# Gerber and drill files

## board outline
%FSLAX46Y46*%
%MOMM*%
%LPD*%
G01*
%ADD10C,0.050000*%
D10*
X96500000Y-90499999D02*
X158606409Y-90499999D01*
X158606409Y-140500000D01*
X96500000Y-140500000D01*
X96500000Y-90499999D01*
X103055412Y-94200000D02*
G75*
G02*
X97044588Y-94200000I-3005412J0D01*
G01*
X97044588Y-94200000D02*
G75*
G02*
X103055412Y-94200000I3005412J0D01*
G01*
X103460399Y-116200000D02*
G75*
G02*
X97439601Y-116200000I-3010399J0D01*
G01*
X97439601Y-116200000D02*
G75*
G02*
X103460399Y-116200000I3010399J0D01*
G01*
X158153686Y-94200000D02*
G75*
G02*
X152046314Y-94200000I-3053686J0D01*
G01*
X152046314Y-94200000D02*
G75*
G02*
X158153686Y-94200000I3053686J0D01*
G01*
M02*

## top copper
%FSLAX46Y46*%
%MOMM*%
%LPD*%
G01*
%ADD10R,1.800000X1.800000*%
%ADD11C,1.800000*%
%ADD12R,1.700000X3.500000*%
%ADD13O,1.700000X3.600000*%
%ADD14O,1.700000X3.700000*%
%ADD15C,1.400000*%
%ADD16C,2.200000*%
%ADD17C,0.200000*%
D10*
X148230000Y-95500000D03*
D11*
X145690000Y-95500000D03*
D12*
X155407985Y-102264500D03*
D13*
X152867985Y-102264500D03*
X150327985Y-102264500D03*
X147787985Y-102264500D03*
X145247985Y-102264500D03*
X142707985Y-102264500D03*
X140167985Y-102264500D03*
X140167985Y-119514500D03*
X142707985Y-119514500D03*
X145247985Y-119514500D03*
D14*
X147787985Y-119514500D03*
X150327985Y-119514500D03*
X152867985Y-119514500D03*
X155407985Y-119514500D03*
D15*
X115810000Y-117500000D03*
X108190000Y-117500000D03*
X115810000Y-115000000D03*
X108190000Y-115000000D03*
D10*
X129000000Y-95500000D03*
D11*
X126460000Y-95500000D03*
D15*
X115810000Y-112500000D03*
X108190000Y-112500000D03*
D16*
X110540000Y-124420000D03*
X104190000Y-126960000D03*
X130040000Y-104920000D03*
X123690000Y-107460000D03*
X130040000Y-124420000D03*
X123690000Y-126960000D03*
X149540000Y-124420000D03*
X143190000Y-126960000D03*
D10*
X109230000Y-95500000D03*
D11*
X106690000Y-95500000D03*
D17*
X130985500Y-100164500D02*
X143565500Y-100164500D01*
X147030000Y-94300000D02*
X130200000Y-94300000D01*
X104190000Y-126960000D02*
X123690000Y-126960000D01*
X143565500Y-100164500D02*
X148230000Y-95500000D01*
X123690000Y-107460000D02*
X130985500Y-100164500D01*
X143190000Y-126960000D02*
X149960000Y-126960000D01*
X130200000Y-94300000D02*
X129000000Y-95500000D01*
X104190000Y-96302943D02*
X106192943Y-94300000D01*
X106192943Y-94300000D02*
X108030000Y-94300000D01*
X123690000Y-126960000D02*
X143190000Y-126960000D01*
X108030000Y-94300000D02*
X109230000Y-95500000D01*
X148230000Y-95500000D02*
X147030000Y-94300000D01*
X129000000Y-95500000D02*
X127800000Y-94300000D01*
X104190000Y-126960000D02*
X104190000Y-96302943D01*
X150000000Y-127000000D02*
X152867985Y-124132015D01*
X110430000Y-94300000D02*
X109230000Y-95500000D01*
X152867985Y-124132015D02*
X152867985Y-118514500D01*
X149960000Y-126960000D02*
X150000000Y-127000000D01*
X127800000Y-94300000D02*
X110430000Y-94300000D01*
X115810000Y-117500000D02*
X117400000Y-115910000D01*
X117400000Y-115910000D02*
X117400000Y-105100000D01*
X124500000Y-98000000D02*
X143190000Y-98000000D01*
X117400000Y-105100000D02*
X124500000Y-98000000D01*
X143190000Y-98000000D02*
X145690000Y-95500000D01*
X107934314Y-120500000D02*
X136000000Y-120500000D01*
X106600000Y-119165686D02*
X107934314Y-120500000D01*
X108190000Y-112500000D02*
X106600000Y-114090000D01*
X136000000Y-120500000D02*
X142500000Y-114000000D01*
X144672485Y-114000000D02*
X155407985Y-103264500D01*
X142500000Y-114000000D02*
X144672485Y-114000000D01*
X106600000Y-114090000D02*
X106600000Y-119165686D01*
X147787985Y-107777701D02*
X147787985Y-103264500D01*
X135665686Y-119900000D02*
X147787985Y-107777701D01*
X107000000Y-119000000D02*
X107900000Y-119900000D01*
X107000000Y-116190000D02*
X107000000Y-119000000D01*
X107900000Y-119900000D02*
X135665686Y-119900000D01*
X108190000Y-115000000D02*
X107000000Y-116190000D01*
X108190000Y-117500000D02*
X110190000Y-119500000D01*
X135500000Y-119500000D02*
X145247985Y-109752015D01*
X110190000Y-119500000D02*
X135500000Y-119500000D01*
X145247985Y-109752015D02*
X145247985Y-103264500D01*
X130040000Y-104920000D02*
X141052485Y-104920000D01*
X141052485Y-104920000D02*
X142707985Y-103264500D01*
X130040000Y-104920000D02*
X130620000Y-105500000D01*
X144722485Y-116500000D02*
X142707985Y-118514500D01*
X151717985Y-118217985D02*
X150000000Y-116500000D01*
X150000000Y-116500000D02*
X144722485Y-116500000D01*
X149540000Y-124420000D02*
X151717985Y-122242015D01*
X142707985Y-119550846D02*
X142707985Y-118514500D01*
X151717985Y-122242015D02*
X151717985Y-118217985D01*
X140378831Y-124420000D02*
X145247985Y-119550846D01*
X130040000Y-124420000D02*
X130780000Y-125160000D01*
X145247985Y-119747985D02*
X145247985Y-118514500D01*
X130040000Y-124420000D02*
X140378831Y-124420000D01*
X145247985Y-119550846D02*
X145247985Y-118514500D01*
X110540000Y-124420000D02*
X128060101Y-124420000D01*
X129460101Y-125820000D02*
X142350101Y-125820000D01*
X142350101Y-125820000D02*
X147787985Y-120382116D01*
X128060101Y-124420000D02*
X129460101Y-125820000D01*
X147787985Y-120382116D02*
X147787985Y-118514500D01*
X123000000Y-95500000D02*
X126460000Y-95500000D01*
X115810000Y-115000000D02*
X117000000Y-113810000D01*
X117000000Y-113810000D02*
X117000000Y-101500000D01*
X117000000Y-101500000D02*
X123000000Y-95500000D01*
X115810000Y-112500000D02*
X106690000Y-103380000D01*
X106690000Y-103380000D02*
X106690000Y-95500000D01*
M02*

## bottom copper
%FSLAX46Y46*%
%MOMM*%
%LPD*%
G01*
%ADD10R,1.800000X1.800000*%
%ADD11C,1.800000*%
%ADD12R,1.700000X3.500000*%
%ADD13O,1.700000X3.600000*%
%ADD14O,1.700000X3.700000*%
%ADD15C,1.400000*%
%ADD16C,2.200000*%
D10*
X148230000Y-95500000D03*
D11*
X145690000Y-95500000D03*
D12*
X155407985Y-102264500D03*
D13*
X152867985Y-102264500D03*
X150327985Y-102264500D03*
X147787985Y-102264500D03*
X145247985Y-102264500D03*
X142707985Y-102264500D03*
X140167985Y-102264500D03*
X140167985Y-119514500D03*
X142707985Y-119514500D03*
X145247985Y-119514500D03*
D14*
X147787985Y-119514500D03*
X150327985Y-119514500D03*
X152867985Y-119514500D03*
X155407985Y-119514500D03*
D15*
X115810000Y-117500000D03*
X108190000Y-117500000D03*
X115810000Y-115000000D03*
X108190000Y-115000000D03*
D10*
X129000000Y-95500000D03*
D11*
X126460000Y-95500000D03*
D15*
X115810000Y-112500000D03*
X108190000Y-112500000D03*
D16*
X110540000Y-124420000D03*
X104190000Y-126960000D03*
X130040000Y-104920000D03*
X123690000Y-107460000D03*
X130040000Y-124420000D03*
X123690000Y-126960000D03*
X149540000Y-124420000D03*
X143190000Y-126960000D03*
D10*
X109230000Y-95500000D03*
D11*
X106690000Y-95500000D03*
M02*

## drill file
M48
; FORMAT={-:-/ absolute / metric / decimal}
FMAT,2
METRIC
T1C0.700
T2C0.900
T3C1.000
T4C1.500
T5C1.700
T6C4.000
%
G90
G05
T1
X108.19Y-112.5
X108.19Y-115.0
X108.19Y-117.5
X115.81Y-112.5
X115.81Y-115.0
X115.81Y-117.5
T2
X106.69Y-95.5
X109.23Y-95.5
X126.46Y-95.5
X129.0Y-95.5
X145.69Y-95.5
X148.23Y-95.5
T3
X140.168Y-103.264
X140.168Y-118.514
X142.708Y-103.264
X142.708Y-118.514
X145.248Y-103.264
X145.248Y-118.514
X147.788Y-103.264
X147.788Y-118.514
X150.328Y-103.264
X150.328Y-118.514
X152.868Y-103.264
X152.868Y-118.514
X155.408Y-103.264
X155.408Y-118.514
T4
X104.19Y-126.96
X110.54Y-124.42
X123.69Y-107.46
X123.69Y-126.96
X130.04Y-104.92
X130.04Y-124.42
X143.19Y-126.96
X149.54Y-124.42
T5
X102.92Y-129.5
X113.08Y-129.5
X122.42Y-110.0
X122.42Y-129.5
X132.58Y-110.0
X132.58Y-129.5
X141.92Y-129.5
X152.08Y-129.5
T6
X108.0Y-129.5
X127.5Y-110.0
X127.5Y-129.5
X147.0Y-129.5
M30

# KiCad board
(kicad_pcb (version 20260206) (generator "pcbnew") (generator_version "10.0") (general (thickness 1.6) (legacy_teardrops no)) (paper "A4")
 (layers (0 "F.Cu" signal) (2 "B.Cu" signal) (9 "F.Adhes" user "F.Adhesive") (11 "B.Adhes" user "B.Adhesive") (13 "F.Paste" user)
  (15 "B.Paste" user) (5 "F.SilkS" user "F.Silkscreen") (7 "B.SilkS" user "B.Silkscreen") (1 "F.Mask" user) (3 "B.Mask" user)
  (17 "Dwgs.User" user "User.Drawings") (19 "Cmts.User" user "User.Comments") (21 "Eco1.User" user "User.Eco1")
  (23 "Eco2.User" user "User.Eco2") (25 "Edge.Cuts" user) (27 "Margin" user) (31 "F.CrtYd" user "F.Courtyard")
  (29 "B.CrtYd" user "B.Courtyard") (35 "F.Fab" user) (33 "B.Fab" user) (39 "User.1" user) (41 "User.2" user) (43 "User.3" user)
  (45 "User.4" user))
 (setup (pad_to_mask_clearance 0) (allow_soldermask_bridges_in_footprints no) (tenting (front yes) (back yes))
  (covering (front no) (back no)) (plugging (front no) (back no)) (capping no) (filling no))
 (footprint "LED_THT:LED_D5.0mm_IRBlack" (layer "F.Cu") (at 148.23 95.5 180)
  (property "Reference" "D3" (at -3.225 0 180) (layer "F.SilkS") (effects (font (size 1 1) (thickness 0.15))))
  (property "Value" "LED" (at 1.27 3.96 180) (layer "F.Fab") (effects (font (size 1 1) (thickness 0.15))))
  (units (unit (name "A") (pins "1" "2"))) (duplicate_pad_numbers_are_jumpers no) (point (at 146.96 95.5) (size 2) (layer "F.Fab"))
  (pad "1" thru_hole rect (at 0 0 180) (size 1.8 1.8) (drill 0.9) (layers "*.Cu" "*.Mask") (remove_unused_layers no) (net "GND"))
  (pad "2" thru_hole circle (at 2.54 0 180) (size 1.8 1.8) (drill 0.9) (layers "*.Cu" "*.Mask") (remove_unused_layers no) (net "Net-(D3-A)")))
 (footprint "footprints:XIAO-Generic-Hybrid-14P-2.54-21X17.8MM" (layer "F.Cu") (at 147.787985 110.8895 -90)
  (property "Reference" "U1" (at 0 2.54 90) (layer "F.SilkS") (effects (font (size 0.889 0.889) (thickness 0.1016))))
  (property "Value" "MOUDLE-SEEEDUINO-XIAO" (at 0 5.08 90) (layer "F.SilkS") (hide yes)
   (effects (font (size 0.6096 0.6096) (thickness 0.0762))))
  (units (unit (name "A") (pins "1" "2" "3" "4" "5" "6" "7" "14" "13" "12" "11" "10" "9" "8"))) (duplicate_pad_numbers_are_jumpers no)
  (pad "1" thru_hole rect (at -7.625 -7.62 270) (size 3.5 1.7) (drill 1 (offset -1 0)) (layers "*.Cu" "*.Mask") (remove_unused_layers no)
   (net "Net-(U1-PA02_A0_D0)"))
  (pad "2" thru_hole oval (at -7.625 -5.08 270) (size 3.6 1.7) (drill 1 (offset -1 0)) (layers "*.Cu" "*.Mask") (remove_unused_layers no)
   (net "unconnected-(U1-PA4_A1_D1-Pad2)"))
  (pad "3" thru_hole oval (at -7.625 -2.54 270) (size 3.6 1.7) (drill 1 (offset -1 0)) (layers "*.Cu" "*.Mask") (remove_unused_layers no)
   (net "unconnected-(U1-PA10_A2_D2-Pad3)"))
  (pad "4" thru_hole oval (at -7.625 0 270) (size 3.6 1.7) (drill 1 (offset -1 0)) (layers "*.Cu" "*.Mask") (remove_unused_layers no)
   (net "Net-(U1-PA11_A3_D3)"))
  (pad "5" thru_hole oval (at -7.625 2.54 270) (size 3.6 1.7) (drill 1 (offset -1 0)) (layers "*.Cu" "*.Mask") (remove_unused_layers no)
   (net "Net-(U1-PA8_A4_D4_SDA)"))
  (pad "6" thru_hole oval (at -7.625 5.08 90) (size 3.6 1.7) (drill 1 (offset 1 0)) (layers "*.Cu" "*.Mask") (remove_unused_layers no)
   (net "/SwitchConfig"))
  (pad "7" thru_hole oval (at -7.625 7.62 270) (size 3.6 1.7) (drill 1 (offset -1 0)) (layers "*.Cu" "*.Mask") (remove_unused_layers no)
   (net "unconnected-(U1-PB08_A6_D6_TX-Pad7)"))
  (pad "8" thru_hole oval (at 7.625 7.62 270) (size 3.6 1.7) (drill 1 (offset 1 0)) (layers "*.Cu" "*.Mask") (remove_unused_layers no)
   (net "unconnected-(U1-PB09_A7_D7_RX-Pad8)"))
  (pad "9" thru_hole oval (at 7.625 5.08 270) (size 3.6 1.7) (drill 1 (offset 1 0)) (layers "*.Cu" "*.Mask") (remove_unused_layers no)
   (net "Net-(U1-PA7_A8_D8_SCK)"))
  (pad "10" thru_hole oval (at 7.625 2.54 270) (size 3.6 1.7) (drill 1 (offset 1 0)) (layers "*.Cu" "*.Mask") (remove_unused_layers no)
   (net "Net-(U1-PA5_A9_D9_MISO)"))
  (pad "11" thru_hole oval (at 7.625 0 270) (size 3.7 1.7) (drill 1 (offset 1 0)) (layers "*.Cu" "*.Mask") (remove_unused_layers no)
   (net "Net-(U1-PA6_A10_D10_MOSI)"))
  (pad "12" thru_hole oval (at 7.625 -2.54 270) (size 3.7 1.7) (drill 1 (offset 1 0)) (layers "*.Cu" "*.Mask") (remove_unused_layers no)
   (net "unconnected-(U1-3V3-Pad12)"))
  (pad "13" thru_hole oval (at 7.625 -5.08 270) (size 3.7 1.7) (drill 1 (offset 1 0)) (layers "*.Cu" "*.Mask") (remove_unused_layers no)
   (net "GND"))
  (pad "14" thru_hole oval (at 7.625 -7.62 270) (size 3.7 1.7) (drill 1 (offset 1 0)) (layers "*.Cu" "*.Mask") (remove_unused_layers no)
   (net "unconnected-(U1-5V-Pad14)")))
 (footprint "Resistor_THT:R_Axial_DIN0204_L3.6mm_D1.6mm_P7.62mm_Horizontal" (layer "F.Cu") (at 115.81 117.5 180)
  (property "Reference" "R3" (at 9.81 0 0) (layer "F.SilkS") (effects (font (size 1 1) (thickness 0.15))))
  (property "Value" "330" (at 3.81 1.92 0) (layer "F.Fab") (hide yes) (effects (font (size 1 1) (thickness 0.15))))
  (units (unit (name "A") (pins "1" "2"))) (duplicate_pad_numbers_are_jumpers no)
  (pad "1" thru_hole circle (at 0 0 180) (size 1.4 1.4) (drill 0.7) (layers "*.Cu" "*.Mask") (remove_unused_layers no) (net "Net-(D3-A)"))
  (pad "2" thru_hole circle (at 7.62 0 180) (size 1.4 1.4) (drill 0.7) (layers "*.Cu" "*.Mask") (remove_unused_layers no)
   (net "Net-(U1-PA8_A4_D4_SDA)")))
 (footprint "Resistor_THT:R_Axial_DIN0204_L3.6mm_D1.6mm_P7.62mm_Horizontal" (layer "F.Cu") (at 115.81 115 180)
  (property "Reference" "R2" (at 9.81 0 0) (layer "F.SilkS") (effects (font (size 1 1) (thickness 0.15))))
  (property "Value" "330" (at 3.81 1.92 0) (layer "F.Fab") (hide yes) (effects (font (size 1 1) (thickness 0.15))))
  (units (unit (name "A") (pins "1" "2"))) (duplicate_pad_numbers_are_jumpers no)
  (pad "1" thru_hole circle (at 0 0 180) (size 1.4 1.4) (drill 0.7) (layers "*.Cu" "*.Mask") (remove_unused_layers no) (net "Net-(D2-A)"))
  (pad "2" thru_hole circle (at 7.62 0 180) (size 1.4 1.4) (drill 0.7) (layers "*.Cu" "*.Mask") (remove_unused_layers no)
   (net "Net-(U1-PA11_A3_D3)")))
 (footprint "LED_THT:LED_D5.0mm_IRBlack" (layer "F.Cu") (at 129 95.5 180)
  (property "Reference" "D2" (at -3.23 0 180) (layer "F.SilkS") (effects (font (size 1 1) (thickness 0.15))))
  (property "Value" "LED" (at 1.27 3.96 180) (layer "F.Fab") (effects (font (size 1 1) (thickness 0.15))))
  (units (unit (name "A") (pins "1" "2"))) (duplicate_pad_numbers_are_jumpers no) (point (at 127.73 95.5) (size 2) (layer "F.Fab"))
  (pad "1" thru_hole rect (at 0 0 180) (size 1.8 1.8) (drill 0.9) (layers "*.Cu" "*.Mask") (remove_unused_layers no) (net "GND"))
  (pad "2" thru_hole circle (at 2.54 0 180) (size 1.8 1.8) (drill 0.9) (layers "*.Cu" "*.Mask") (remove_unused_layers no) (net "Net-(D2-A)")))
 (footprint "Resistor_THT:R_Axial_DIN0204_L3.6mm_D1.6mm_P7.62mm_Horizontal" (layer "F.Cu") (at 115.81 112.5 180)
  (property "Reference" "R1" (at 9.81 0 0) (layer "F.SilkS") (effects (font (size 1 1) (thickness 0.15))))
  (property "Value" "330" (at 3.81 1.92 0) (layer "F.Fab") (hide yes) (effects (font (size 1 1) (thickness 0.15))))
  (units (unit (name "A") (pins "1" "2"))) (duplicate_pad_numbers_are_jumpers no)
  (pad "1" thru_hole circle (at 0 0 180) (size 1.4 1.4) (drill 0.7) (layers "*.Cu" "*.Mask") (remove_unused_layers no) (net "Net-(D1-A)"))
  (pad "2" thru_hole circle (at 7.62 0 180) (size 1.4 1.4) (drill 0.7) (layers "*.Cu" "*.Mask") (remove_unused_layers no)
   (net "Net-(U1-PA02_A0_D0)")))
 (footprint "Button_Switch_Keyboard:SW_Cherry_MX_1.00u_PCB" (layer "F.Cu") (at 110.54 124.42)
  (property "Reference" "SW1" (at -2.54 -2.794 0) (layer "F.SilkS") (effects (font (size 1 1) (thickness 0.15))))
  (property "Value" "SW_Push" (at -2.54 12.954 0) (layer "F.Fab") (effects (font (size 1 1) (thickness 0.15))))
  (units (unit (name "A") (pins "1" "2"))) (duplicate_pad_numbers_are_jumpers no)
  (pad "" np_thru_hole circle (at -7.62 5.08) (size 1.7 1.7) (drill 1.7) (layers "*.Cu" "*.Mask"))
  (pad "" np_thru_hole circle (at -2.54 5.08) (size 4 4) (drill 4) (layers "*.Cu" "*.Mask"))
  (pad "" np_thru_hole circle (at 2.54 5.08) (size 1.7 1.7) (drill 1.7) (layers "*.Cu" "*.Mask"))
  (pad "1" thru_hole circle (at 0 0) (size 2.2 2.2) (drill 1.5) (layers "*.Cu" "*.Mask") (remove_unused_layers no)
   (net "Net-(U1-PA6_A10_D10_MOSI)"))
  (pad "2" thru_hole circle (at -6.35 2.54) (size 2.2 2.2) (drill 1.5) (layers "*.Cu" "*.Mask") (remove_unused_layers no) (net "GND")))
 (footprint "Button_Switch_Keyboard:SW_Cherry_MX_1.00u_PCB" (layer "F.Cu") (at 130.04 104.92)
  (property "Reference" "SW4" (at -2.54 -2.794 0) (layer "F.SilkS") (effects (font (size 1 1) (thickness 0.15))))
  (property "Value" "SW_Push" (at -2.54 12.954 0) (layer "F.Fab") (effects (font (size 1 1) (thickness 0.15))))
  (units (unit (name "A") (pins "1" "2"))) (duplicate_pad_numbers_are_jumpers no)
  (pad "" np_thru_hole circle (at -7.62 5.08) (size 1.7 1.7) (drill 1.7) (layers "*.Cu" "*.Mask"))
  (pad "" np_thru_hole circle (at -2.54 5.08) (size 4 4) (drill 4) (layers "*.Cu" "*.Mask"))
  (pad "" np_thru_hole circle (at 2.54 5.08) (size 1.7 1.7) (drill 1.7) (layers "*.Cu" "*.Mask"))
  (pad "1" thru_hole circle (at 0 0) (size 2.2 2.2) (drill 1.5) (layers "*.Cu" "*.Mask") (remove_unused_layers no) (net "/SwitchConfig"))
  (pad "2" thru_hole circle (at -6.35 2.54) (size 2.2 2.2) (drill 1.5) (layers "*.Cu" "*.Mask") (remove_unused_layers no) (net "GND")))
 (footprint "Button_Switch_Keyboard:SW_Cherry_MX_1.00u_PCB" (layer "F.Cu") (at 130.04 124.42)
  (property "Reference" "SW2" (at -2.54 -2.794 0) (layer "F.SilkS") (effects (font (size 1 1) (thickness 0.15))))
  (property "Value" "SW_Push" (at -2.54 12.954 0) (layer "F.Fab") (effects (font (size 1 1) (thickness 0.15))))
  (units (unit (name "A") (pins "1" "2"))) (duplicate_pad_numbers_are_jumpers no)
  (pad "" np_thru_hole circle (at -7.62 5.08) (size 1.7 1.7) (drill 1.7) (layers "*.Cu" "*.Mask"))
  (pad "" np_thru_hole circle (at -2.54 5.08) (size 4 4) (drill 4) (layers "*.Cu" "*.Mask"))
  (pad "" np_thru_hole circle (at 2.54 5.08) (size 1.7 1.7) (drill 1.7) (layers "*.Cu" "*.Mask"))
  (pad "1" thru_hole circle (at 0 0) (size 2.2 2.2) (drill 1.5) (layers "*.Cu" "*.Mask") (remove_unused_layers no)
   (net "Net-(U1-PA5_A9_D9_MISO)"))
  (pad "2" thru_hole circle (at -6.35 2.54) (size 2.2 2.2) (drill 1.5) (layers "*.Cu" "*.Mask") (remove_unused_layers no) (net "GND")))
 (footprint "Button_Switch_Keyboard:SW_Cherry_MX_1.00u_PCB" (layer "F.Cu") (at 149.54 124.42)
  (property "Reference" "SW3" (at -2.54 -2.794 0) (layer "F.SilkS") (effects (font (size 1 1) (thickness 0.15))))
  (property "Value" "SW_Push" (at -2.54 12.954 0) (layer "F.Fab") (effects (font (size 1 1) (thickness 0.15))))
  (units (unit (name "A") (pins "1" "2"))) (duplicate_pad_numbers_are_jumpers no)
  (pad "" np_thru_hole circle (at -7.62 5.08) (size 1.7 1.7) (drill 1.7) (layers "*.Cu" "*.Mask"))
  (pad "" np_thru_hole circle (at -2.54 5.08) (size 4 4) (drill 4) (layers "*.Cu" "*.Mask"))
  (pad "" np_thru_hole circle (at 2.54 5.08) (size 1.7 1.7) (drill 1.7) (layers "*.Cu" "*.Mask"))
  (pad "1" thru_hole circle (at 0 0) (size 2.2 2.2) (drill 1.5) (layers "*.Cu" "*.Mask") (remove_unused_layers no)
   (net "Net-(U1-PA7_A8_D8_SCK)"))
  (pad "2" thru_hole circle (at -6.35 2.54) (size 2.2 2.2) (drill 1.5) (layers "*.Cu" "*.Mask") (remove_unused_layers no) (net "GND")))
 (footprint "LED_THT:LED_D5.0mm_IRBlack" (layer "F.Cu") (at 109.23 95.5 180)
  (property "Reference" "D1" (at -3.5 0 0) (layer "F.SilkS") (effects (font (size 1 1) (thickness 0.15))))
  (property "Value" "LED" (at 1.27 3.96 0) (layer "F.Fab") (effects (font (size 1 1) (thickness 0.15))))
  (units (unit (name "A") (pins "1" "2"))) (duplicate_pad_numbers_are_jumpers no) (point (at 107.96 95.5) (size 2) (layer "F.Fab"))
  (pad "1" thru_hole rect (at 0 0 180) (size 1.8 1.8) (drill 0.9) (layers "*.Cu" "*.Mask") (remove_unused_layers no) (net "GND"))
  (pad "2" thru_hole circle (at 2.54 0 180) (size 1.8 1.8) (drill 0.9) (layers "*.Cu" "*.Mask") (remove_unused_layers no) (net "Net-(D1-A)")))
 (gr_rect (start 96.5 90.499999) (end 158.606409 140.5) (stroke (width 0.05) (type default)) (fill no) (layer "Edge.Cuts"))
 (gr_circle (center 100.05 94.2) (end 102.15 96.35) (stroke (width 0.05) (type default)) (fill no) (layer "Edge.Cuts"))
 (gr_circle (center 100.45 116.2) (end 102.45 113.95) (stroke (width 0.05) (type default)) (fill no) (layer "Edge.Cuts"))
 (gr_circle (center 155.1 94.2) (end 157.45 92.25) (stroke (width 0.05) (type default)) (fill no) (layer "Edge.Cuts"))
 (segment (start 130.9855 100.1645) (end 143.5655 100.1645) (width 0.2) (layer "F.Cu") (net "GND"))
 (segment (start 147.03 94.3) (end 130.2 94.3) (width 0.2) (layer "F.Cu") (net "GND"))
 (segment (start 104.19 126.96) (end 123.69 126.96) (width 0.2) (layer "F.Cu") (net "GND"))
 (segment (start 143.5655 100.1645) (end 148.23 95.5) (width 0.2) (layer "F.Cu") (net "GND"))
 (segment (start 123.69 107.46) (end 130.9855 100.1645) (width 0.2) (layer "F.Cu") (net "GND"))
 (segment (start 143.19 126.96) (end 149.96 126.96) (width 0.2) (layer "F.Cu") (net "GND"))
 (segment (start 130.2 94.3) (end 129 95.5) (width 0.2) (layer "F.Cu") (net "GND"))
 (segment (start 104.19 96.302943) (end 106.192943 94.3) (width 0.2) (layer "F.Cu") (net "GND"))
 (segment (start 106.192943 94.3) (end 108.03 94.3) (width 0.2) (layer "F.Cu") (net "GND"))
 (segment (start 123.69 126.96) (end 143.19 126.96) (width 0.2) (layer "F.Cu") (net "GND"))
 (segment (start 108.03 94.3) (end 109.23 95.5) (width 0.2) (layer "F.Cu") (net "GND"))
 (segment (start 148.23 95.5) (end 147.03 94.3) (width 0.2) (layer "F.Cu") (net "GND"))
 (segment (start 129 95.5) (end 127.8 94.3) (width 0.2) (layer "F.Cu") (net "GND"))
 (segment (start 104.19 126.96) (end 104.19 96.302943) (width 0.2) (layer "F.Cu") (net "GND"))
 (segment (start 150 127) (end 152.867985 124.132015) (width 0.2) (layer "F.Cu") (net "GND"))
 (segment (start 110.43 94.3) (end 109.23 95.5) (width 0.2) (layer "F.Cu") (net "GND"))
 (segment (start 152.867985 124.132015) (end 152.867985 118.5145) (width 0.2) (layer "F.Cu") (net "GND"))
 (segment (start 149.96 126.96) (end 150 127) (width 0.2) (layer "F.Cu") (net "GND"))
 (segment (start 127.8 94.3) (end 110.43 94.3) (width 0.2) (layer "F.Cu") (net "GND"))
 (segment (start 115.81 117.5) (end 117.4 115.91) (width 0.2) (layer "F.Cu") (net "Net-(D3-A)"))
 (segment (start 117.4 115.91) (end 117.4 105.1) (width 0.2) (layer "F.Cu") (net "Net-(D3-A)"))
 (segment (start 124.5 98) (end 143.19 98) (width 0.2) (layer "F.Cu") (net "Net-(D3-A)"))
 (segment (start 117.4 105.1) (end 124.5 98) (width 0.2) (layer "F.Cu") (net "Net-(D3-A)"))
 (segment (start 143.19 98) (end 145.69 95.5) (width 0.2) (layer "F.Cu") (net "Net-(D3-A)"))
 (segment (start 107.934314 120.5) (end 136 120.5) (width 0.2) (layer "F.Cu") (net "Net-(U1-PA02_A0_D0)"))
 (segment (start 106.6 119.165686) (end 107.934314 120.5) (width 0.2) (layer "F.Cu") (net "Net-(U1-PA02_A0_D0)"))
 (segment (start 108.19 112.5) (end 106.6 114.09) (width 0.2) (layer "F.Cu") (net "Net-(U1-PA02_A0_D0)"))
 (segment (start 136 120.5) (end 142.5 114) (width 0.2) (layer "F.Cu") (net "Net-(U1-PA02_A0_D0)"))
 (segment (start 144.672485 114) (end 155.407985 103.2645) (width 0.2) (layer "F.Cu") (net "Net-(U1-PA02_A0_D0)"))
 (segment (start 142.5 114) (end 144.672485 114) (width 0.2) (layer "F.Cu") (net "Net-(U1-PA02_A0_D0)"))
 (segment (start 106.6 114.09) (end 106.6 119.165686) (width 0.2) (layer "F.Cu") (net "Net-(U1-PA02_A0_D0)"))
 (segment (start 147.787985 107.777701) (end 147.787985 103.2645) (width 0.2) (layer "F.Cu") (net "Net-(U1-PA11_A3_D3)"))
 (segment (start 135.665686 119.9) (end 147.787985 107.777701) (width 0.2) (layer "F.Cu") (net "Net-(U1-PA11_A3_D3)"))
 (segment (start 107 119) (end 107.9 119.9) (width 0.2) (layer "F.Cu") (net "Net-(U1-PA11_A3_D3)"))
 (segment (start 107 116.19) (end 107 119) (width 0.2) (layer "F.Cu") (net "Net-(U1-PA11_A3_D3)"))
 (segment (start 107.9 119.9) (end 135.665686 119.9) (width 0.2) (layer "F.Cu") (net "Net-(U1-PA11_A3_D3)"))
 (segment (start 108.19 115) (end 107 116.19) (width 0.2) (layer "F.Cu") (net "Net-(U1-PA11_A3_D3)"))
 (segment (start 108.19 117.5) (end 110.19 119.5) (width 0.2) (layer "F.Cu") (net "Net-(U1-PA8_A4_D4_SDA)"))
 (segment (start 135.5 119.5) (end 145.247985 109.752015) (width 0.2) (layer "F.Cu") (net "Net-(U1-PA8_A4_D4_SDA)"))
 (segment (start 110.19 119.5) (end 135.5 119.5) (width 0.2) (layer "F.Cu") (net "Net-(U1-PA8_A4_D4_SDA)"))
 (segment (start 145.247985 109.752015) (end 145.247985 103.2645) (width 0.2) (layer "F.Cu") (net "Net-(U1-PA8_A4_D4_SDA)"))
 (segment (start 130.04 104.92) (end 141.052485 104.92) (width 0.2) (layer "F.Cu") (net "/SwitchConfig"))
 (segment (start 141.052485 104.92) (end 142.707985 103.2645) (width 0.2) (layer "F.Cu") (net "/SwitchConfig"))
 (segment (start 130.04 104.92) (end 130.62 105.5) (width 0.2) (layer "F.Cu") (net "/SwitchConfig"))
 (segment (start 144.722485 116.5) (end 142.707985 118.5145) (width 0.2) (layer "F.Cu") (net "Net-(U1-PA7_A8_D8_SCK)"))
 (segment (start 151.717985 118.217985) (end 150 116.5) (width 0.2) (layer "F.Cu") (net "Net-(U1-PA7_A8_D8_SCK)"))
 (segment (start 150 116.5) (end 144.722485 116.5) (width 0.2) (layer "F.Cu") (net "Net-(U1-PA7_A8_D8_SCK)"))
 (segment (start 149.54 124.42) (end 151.717985 122.242015) (width 0.2) (layer "F.Cu") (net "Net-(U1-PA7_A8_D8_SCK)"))
 (segment (start 142.707985 119.550846) (end 142.707985 118.5145) (width 0.2) (layer "F.Cu") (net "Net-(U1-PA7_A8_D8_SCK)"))
 (segment (start 151.717985 122.242015) (end 151.717985 118.217985) (width 0.2) (layer "F.Cu") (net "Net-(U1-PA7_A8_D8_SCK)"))
 (segment (start 140.378831 124.42) (end 145.247985 119.550846) (width 0.2) (layer "F.Cu") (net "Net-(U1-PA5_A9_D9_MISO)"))
 (segment (start 130.04 124.42) (end 130.78 125.16) (width 0.2) (layer "F.Cu") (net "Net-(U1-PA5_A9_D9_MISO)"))
 (segment (start 145.247985 119.747985) (end 145.247985 118.5145) (width 0.2) (layer "F.Cu") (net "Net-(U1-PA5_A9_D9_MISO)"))
 (segment (start 130.04 124.42) (end 140.378831 124.42) (width 0.2) (layer "F.Cu") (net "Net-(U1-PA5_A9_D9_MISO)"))
 (segment (start 145.247985 119.550846) (end 145.247985 118.5145) (width 0.2) (layer "F.Cu") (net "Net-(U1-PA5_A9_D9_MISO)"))
 (segment (start 110.54 124.42) (end 128.060101 124.42) (width 0.2) (layer "F.Cu") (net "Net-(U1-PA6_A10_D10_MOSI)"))
 (segment (start 129.460101 125.82) (end 142.350101 125.82) (width 0.2) (layer "F.Cu") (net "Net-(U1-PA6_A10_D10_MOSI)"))
 (segment (start 142.350101 125.82) (end 147.787985 120.382116) (width 0.2) (layer "F.Cu") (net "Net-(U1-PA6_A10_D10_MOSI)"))
 (segment (start 128.060101 124.42) (end 129.460101 125.82) (width 0.2) (layer "F.Cu") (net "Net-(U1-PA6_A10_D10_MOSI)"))
 (segment (start 147.787985 120.382116) (end 147.787985 118.5145) (width 0.2) (layer "F.Cu") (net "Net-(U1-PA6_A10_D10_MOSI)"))
 (segment (start 123 95.5) (end 126.46 95.5) (width 0.2) (layer "F.Cu") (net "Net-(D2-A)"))
 (segment (start 115.81 115) (end 117 113.81) (width 0.2) (layer "F.Cu") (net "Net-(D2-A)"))
 (segment (start 117 113.81) (end 117 101.5) (width 0.2) (layer "F.Cu") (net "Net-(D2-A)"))
 (segment (start 117 101.5) (end 123 95.5) (width 0.2) (layer "F.Cu") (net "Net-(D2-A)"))
 (segment (start 115.81 112.5) (end 106.69 103.38) (width 0.2) (layer "F.Cu") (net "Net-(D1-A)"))
 (segment (start 106.69 103.38) (end 106.69 95.5) (width 0.2) (layer "F.Cu") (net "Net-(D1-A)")))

